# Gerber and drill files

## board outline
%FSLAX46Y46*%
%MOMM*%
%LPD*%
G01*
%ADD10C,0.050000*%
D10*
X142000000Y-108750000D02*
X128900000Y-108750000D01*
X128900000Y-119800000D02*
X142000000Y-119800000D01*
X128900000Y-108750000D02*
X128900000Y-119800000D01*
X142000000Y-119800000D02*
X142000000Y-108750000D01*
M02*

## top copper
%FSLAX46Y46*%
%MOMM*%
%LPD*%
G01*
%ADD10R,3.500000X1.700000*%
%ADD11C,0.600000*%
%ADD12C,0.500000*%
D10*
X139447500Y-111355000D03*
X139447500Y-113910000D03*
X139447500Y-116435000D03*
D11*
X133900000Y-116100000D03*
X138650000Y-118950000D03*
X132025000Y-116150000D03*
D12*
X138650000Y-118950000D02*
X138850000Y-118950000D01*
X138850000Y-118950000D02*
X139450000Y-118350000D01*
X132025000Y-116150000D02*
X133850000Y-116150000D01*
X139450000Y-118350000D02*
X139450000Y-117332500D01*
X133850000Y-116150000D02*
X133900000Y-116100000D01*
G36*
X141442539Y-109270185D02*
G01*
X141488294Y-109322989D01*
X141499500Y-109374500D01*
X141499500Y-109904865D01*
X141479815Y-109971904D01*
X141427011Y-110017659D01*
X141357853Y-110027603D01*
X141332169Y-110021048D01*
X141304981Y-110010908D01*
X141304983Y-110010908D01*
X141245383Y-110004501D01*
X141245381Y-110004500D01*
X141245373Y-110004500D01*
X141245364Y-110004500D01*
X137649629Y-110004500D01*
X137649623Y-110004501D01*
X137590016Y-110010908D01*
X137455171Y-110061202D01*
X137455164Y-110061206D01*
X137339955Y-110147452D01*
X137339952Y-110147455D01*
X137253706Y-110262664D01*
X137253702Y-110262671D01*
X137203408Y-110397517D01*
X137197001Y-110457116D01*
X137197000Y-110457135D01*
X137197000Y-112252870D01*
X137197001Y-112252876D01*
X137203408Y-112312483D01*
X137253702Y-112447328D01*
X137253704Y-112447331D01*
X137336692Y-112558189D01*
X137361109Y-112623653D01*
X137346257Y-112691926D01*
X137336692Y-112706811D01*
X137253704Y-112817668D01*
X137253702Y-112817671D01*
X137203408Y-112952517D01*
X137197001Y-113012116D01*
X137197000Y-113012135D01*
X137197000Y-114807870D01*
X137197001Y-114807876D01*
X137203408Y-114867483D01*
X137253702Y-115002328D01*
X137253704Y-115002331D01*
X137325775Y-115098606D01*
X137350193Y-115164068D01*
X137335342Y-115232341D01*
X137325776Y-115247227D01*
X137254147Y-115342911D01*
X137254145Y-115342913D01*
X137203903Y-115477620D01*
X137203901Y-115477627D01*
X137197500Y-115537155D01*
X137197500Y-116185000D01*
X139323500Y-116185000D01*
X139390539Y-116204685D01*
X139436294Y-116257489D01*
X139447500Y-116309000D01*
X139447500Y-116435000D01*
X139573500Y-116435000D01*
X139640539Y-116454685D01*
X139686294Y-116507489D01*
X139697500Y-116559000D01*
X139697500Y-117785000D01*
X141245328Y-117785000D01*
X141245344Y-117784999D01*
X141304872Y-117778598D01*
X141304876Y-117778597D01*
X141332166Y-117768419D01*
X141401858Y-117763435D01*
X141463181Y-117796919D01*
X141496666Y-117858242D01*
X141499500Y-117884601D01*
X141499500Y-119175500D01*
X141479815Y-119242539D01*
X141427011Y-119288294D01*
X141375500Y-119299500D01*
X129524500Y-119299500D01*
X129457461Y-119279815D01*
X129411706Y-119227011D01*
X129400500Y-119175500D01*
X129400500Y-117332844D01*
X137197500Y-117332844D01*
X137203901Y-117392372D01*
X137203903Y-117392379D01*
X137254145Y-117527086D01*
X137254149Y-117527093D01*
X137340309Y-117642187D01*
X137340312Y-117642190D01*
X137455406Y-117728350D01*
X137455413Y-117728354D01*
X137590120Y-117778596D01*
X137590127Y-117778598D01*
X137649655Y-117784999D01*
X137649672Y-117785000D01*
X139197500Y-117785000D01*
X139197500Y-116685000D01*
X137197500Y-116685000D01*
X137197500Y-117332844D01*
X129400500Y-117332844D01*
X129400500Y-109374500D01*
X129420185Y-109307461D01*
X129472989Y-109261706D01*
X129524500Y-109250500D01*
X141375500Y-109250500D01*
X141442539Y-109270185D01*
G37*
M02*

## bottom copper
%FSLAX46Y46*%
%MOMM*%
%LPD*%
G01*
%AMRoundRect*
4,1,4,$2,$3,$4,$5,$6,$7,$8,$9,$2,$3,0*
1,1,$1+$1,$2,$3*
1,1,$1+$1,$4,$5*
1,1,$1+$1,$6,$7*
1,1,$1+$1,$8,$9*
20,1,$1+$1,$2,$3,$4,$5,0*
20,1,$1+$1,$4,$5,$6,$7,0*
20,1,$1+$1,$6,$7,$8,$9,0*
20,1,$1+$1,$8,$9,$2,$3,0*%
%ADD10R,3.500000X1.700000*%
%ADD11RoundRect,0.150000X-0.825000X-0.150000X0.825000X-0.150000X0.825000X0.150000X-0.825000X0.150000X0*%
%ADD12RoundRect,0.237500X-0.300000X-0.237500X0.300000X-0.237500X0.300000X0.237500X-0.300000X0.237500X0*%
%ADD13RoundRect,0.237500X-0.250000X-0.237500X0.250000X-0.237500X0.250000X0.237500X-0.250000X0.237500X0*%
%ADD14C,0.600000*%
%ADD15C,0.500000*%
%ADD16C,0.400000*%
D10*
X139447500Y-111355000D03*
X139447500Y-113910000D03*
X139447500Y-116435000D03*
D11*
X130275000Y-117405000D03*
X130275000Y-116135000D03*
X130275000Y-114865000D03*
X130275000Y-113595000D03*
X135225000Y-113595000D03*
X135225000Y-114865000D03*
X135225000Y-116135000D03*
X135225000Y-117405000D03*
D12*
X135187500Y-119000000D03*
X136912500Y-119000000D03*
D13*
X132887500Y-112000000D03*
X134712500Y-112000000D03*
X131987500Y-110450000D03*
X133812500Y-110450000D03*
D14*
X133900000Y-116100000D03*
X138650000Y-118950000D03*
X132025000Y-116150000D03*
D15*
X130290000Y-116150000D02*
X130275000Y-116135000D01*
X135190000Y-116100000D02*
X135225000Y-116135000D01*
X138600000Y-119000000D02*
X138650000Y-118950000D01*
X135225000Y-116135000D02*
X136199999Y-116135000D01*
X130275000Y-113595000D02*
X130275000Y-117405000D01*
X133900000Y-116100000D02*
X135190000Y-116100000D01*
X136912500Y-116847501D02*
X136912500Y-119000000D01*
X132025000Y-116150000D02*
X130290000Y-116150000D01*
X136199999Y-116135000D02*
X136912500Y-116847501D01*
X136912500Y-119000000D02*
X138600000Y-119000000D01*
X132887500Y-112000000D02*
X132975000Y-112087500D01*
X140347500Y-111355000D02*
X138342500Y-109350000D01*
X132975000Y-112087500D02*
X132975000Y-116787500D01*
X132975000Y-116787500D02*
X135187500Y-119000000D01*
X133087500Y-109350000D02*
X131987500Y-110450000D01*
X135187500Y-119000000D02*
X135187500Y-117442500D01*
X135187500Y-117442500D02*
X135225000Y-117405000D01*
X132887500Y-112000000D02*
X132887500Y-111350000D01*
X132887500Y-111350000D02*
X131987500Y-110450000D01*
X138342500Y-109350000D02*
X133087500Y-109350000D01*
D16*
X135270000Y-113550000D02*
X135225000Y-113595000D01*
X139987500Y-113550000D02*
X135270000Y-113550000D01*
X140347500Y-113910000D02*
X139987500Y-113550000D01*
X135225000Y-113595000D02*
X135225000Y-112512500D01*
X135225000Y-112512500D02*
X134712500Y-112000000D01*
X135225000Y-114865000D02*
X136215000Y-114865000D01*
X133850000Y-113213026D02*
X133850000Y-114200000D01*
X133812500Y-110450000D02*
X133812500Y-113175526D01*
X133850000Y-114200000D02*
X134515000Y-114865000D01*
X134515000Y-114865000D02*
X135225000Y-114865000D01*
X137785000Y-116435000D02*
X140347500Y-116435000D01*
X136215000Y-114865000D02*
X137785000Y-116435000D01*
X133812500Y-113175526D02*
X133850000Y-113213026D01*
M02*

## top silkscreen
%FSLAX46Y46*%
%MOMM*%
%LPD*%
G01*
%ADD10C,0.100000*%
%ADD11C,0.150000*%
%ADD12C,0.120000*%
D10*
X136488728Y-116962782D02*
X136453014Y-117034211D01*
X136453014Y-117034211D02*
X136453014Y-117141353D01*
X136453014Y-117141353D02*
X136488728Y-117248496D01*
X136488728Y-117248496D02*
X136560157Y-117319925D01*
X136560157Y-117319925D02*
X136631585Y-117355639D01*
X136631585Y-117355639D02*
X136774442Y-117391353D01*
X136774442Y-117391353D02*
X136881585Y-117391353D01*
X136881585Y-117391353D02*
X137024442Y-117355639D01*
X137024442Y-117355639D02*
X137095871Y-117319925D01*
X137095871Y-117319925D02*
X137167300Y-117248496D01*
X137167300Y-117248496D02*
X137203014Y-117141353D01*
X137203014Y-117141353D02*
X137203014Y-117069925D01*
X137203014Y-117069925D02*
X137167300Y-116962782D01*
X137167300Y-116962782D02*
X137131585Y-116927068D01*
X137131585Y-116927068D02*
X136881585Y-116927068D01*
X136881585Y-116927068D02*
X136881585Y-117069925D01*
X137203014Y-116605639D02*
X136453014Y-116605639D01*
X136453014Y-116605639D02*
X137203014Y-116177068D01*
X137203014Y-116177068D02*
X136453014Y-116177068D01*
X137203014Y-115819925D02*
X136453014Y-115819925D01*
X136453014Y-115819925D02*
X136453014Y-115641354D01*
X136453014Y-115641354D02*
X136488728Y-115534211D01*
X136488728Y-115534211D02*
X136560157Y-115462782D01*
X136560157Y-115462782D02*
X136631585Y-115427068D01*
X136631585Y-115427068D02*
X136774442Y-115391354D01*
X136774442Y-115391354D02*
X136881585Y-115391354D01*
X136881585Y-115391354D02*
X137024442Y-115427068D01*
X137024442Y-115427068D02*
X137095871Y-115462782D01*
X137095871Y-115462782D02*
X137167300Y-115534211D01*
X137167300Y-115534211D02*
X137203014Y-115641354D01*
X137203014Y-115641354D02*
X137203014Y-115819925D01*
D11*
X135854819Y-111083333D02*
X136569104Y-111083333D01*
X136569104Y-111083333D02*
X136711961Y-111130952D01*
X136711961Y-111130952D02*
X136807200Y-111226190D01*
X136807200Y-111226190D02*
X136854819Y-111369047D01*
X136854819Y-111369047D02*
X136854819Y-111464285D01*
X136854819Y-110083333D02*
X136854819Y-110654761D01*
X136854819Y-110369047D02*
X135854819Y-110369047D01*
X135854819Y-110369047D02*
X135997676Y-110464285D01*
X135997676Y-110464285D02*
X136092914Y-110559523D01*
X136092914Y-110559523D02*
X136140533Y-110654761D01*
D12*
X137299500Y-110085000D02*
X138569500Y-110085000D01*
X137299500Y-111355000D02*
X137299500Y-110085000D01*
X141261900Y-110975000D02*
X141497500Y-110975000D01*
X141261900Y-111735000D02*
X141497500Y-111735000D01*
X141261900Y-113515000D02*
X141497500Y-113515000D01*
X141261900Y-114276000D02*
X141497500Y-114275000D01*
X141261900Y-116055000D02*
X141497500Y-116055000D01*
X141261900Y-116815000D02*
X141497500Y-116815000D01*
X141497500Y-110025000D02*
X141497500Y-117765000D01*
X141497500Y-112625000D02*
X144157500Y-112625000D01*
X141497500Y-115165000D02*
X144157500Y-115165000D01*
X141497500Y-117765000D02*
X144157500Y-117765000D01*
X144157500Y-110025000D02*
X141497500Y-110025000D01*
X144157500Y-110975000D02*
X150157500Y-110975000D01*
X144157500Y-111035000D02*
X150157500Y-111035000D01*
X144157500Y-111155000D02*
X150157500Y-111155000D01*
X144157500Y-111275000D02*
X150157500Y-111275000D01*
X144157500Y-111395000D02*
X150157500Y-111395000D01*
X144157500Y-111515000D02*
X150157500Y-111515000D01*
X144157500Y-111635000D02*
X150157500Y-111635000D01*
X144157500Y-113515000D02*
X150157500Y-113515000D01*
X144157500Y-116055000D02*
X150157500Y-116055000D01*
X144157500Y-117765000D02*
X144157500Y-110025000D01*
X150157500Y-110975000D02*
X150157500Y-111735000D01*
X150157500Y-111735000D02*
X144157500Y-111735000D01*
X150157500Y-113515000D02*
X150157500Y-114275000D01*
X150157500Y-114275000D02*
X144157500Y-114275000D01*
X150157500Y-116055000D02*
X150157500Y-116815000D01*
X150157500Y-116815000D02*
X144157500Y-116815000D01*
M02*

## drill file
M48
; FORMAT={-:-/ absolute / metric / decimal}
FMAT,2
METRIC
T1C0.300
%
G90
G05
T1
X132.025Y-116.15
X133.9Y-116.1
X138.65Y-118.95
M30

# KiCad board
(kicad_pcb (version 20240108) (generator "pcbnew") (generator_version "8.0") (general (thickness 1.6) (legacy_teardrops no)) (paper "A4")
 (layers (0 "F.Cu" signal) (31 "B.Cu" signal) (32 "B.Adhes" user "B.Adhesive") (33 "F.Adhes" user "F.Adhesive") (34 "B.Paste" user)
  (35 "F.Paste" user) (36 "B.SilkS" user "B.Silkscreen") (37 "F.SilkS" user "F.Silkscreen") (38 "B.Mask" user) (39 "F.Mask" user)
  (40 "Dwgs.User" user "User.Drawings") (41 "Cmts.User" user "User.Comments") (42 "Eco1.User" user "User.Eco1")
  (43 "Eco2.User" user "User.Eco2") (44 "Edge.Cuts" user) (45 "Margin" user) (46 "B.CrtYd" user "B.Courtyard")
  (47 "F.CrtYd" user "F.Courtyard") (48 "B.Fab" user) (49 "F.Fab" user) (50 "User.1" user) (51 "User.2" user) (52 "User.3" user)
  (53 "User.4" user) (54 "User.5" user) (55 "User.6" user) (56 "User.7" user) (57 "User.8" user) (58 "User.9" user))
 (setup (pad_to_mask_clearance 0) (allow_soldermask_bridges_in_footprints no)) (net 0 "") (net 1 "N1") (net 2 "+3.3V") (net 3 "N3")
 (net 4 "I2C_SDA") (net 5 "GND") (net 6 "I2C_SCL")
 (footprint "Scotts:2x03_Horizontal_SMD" (layer "F.Cu") (at 140.3475 108.815)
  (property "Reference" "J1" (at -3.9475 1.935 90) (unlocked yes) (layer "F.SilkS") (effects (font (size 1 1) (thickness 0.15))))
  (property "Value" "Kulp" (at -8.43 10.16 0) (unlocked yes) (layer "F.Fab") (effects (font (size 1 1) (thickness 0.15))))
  (fp_line (start -3.048 1.27) (end -1.778 1.27) (stroke (width 0.12) (type solid)) (layer "F.SilkS"))
  (fp_line (start -3.048 2.54) (end -3.048 1.27) (stroke (width 0.12) (type solid)) (layer "F.SilkS"))
  (fp_line (start 0.9144 2.16) (end 1.15 2.16) (stroke (width 0.12) (type solid)) (layer "F.SilkS"))
  (fp_line (start 0.9144 2.92) (end 1.15 2.92) (stroke (width 0.12) (type solid)) (layer "F.SilkS"))
  (fp_line (start 0.9144 4.7) (end 1.15 4.7) (stroke (width 0.12) (type solid)) (layer "F.SilkS"))
  (fp_line (start 0.9144 5.461) (end 1.15 5.46) (stroke (width 0.12) (type solid)) (layer "F.SilkS"))
  (fp_line (start 0.9144 7.24) (end 1.15 7.24) (stroke (width 0.12) (type solid)) (layer "F.SilkS"))
  (fp_line (start 0.9144 8) (end 1.15 8) (stroke (width 0.12) (type solid)) (layer "F.SilkS"))
  (fp_line (start 1.15 1.21) (end 1.15 8.95) (stroke (width 0.12) (type solid)) (layer "F.SilkS"))
  (fp_line (start 1.15 3.81) (end 3.81 3.81) (stroke (width 0.12) (type solid)) (layer "F.SilkS"))
  (fp_line (start 1.15 6.35) (end 3.81 6.35) (stroke (width 0.12) (type solid)) (layer "F.SilkS"))
  (fp_line (start 1.15 8.95) (end 3.81 8.95) (stroke (width 0.12) (type solid)) (layer "F.SilkS"))
  (fp_line (start 3.81 1.21) (end 1.15 1.21) (stroke (width 0.12) (type solid)) (layer "F.SilkS"))
  (fp_line (start 3.81 2.16) (end 9.81 2.16) (stroke (width 0.12) (type solid)) (layer "F.SilkS"))
  (fp_line (start 3.81 2.22) (end 9.81 2.22) (stroke (width 0.12) (type solid)) (layer "F.SilkS"))
  (fp_line (start 3.81 2.34) (end 9.81 2.34) (stroke (width 0.12) (type solid)) (layer "F.SilkS"))
  (fp_line (start 3.81 2.46) (end 9.81 2.46) (stroke (width 0.12) (type solid)) (layer "F.SilkS"))
  (fp_line (start 3.81 2.58) (end 9.81 2.58) (stroke (width 0.12) (type solid)) (layer "F.SilkS"))
  (fp_line (start 3.81 2.7) (end 9.81 2.7) (stroke (width 0.12) (type solid)) (layer "F.SilkS"))
  (fp_line (start 3.81 2.82) (end 9.81 2.82) (stroke (width 0.12) (type solid)) (layer "F.SilkS"))
  (fp_line (start 3.81 4.7) (end 9.81 4.7) (stroke (width 0.12) (type solid)) (layer "F.SilkS"))
  (fp_line (start 3.81 7.24) (end 9.81 7.24) (stroke (width 0.12) (type solid)) (layer "F.SilkS"))
  (fp_line (start 3.81 8.95) (end 3.81 1.21) (stroke (width 0.12) (type solid)) (layer "F.SilkS"))
  (fp_line (start 9.81 2.16) (end 9.81 2.92) (stroke (width 0.12) (type solid)) (layer "F.SilkS"))
  (fp_line (start 9.81 2.92) (end 3.81 2.92) (stroke (width 0.12) (type solid)) (layer "F.SilkS"))
  (fp_line (start 9.81 4.7) (end 9.81 5.46) (stroke (width 0.12) (type solid)) (layer "F.SilkS"))
  (fp_line (start 9.81 5.46) (end 3.81 5.46) (stroke (width 0.12) (type solid)) (layer "F.SilkS"))
  (fp_line (start 9.81 7.24) (end 9.81 8) (stroke (width 0.12) (type solid)) (layer "F.SilkS"))
  (fp_line (start 9.81 8) (end 3.81 8) (stroke (width 0.12) (type solid)) (layer "F.SilkS"))
  (pad "1" smd rect (at 0 2.54) (size 3.5 1.7) (drill (offset -0.9 0)) (layers "F.Cu" "F.Mask") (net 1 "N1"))
  (pad "2" smd rect (at 0 2.54) (size 3.5 1.7) (drill (offset -0.9 0)) (layers "B.Cu" "B.Mask") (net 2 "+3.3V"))
  (pad "3" smd rect (at 0 5.095) (size 3.5 1.7) (drill (offset -0.9 0)) (layers "F.Cu" "F.Mask") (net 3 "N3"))
  (pad "4" smd rect (at 0 5.095) (size 3.5 1.7) (drill (offset -0.9 0)) (layers "B.Cu" "B.Mask") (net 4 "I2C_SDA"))
  (pad "5" smd rect (at 0 7.62) (size 3.5 1.7) (drill (offset -0.9 0)) (layers "F.Cu" "F.Mask") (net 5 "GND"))
  (pad "6" smd rect (at 0 7.62) (size 3.5 1.7) (drill (offset -0.9 0)) (layers "B.Cu" "B.Mask") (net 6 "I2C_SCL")))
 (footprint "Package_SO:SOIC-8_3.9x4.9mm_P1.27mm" (layer "B.Cu") (at 132.75 115.5)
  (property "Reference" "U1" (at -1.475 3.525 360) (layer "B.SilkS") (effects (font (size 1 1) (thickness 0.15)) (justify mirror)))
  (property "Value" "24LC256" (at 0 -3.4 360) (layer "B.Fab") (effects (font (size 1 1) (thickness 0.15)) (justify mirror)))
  (pad "1" smd roundrect (at -2.475 1.905) (size 1.95 0.6) (layers "B.Cu" "B.Paste" "B.Mask") (roundrect_rratio 0.25) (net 5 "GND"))
  (pad "2" smd roundrect (at -2.475 0.635) (size 1.95 0.6) (layers "B.Cu" "B.Paste" "B.Mask") (roundrect_rratio 0.25) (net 5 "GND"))
  (pad "3" smd roundrect (at -2.475 -0.635) (size 1.95 0.6) (layers "B.Cu" "B.Paste" "B.Mask") (roundrect_rratio 0.25) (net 5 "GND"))
  (pad "4" smd roundrect (at -2.475 -1.905) (size 1.95 0.6) (layers "B.Cu" "B.Paste" "B.Mask") (roundrect_rratio 0.25) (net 5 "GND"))
  (pad "5" smd roundrect (at 2.475 -1.905) (size 1.95 0.6) (layers "B.Cu" "B.Paste" "B.Mask") (roundrect_rratio 0.25) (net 4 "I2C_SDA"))
  (pad "6" smd roundrect (at 2.475 -0.635) (size 1.95 0.6) (layers "B.Cu" "B.Paste" "B.Mask") (roundrect_rratio 0.25) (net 6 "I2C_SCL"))
  (pad "7" smd roundrect (at 2.475 0.635) (size 1.95 0.6) (layers "B.Cu" "B.Paste" "B.Mask") (roundrect_rratio 0.25) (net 5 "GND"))
  (pad "8" smd roundrect (at 2.475 1.905) (size 1.95 0.6) (layers "B.Cu" "B.Paste" "B.Mask") (roundrect_rratio 0.25) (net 2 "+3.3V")))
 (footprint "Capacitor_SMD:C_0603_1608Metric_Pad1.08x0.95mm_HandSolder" (layer "B.Cu") (at 136.05 119)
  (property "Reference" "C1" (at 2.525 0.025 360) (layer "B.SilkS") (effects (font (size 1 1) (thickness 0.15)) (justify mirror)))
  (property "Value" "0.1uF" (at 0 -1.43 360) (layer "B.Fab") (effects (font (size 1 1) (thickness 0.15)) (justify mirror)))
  (pad "1" smd roundrect (at -0.8625 0) (size 1.075 0.95) (layers "B.Cu" "B.Paste" "B.Mask") (roundrect_rratio 0.25) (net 2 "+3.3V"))
  (pad "2" smd roundrect (at 0.8625 0) (size 1.075 0.95) (layers "B.Cu" "B.Paste" "B.Mask") (roundrect_rratio 0.25) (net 5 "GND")))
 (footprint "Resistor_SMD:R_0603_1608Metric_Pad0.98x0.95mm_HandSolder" (layer "B.Cu") (at 133.8 112)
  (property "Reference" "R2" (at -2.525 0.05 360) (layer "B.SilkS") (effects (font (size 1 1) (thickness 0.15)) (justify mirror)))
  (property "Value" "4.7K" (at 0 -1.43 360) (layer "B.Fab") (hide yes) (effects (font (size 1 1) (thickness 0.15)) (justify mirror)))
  (pad "1" smd roundrect (at -0.9125 0) (size 0.975 0.95) (layers "B.Cu" "B.Paste" "B.Mask") (roundrect_rratio 0.25) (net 2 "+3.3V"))
  (pad "2" smd roundrect (at 0.9125 0) (size 0.975 0.95) (layers "B.Cu" "B.Paste" "B.Mask") (roundrect_rratio 0.25) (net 4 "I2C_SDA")))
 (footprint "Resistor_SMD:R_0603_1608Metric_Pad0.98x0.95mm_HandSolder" (layer "B.Cu") (at 132.9 110.45)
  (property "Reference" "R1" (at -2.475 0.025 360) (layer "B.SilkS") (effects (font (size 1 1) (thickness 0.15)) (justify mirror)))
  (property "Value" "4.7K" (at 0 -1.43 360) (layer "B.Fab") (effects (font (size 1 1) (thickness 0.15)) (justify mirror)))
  (pad "1" smd roundrect (at -0.9125 0) (size 0.975 0.95) (layers "B.Cu" "B.Paste" "B.Mask") (roundrect_rratio 0.25) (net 2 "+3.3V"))
  (pad "2" smd roundrect (at 0.9125 0) (size 0.975 0.95) (layers "B.Cu" "B.Paste" "B.Mask") (roundrect_rratio 0.25) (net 6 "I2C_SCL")))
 (gr_line (start 142 108.75) (end 128.9 108.75) (stroke (width 0.05) (type default)) (layer "Edge.Cuts"))
 (gr_line (start 128.9 119.8) (end 142 119.8) (stroke (width 0.05) (type default)) (layer "Edge.Cuts"))
 (gr_line (start 128.9 108.75) (end 128.9 119.8) (stroke (width 0.05) (type default)) (layer "Edge.Cuts"))
 (gr_line (start 142 119.8) (end 142 108.75) (stroke (width 0.05) (type default)) (layer "Edge.Cuts"))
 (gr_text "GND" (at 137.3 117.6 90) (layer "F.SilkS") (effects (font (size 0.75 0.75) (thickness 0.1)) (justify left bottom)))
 (segment (start 138.65 118.95) (end 138.85 118.95) (width 0.5) (layer "F.Cu") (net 5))
 (segment (start 138.85 118.95) (end 139.45 118.35) (width 0.5) (layer "F.Cu") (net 5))
 (segment (start 132.025 116.15) (end 133.85 116.15) (width 0.5) (layer "F.Cu") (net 5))
 (segment (start 139.45 118.35) (end 139.45 117.3325) (width 0.5) (layer "F.Cu") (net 5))
 (segment (start 133.85 116.15) (end 133.9 116.1) (width 0.5) (layer "F.Cu") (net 5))
 (via (at 133.9 116.1) (size 0.6) (drill 0.3) (layers "F.Cu" "B.Cu") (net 5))
 (via (at 138.65 118.95) (size 0.6) (drill 0.3) (layers "F.Cu" "B.Cu") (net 5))
 (via (at 132.025 116.15) (size 0.6) (drill 0.3) (layers "F.Cu" "B.Cu") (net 5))
 (segment (start 130.29 116.15) (end 130.275 116.135) (width 0.5) (layer "B.Cu") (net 5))
 (segment (start 135.19 116.1) (end 135.225 116.135) (width 0.5) (layer "B.Cu") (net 5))
 (segment (start 138.6 119) (end 138.65 118.95) (width 0.5) (layer "B.Cu") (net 5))
 (segment (start 135.225 116.135) (end 136.199999 116.135) (width 0.5) (layer "B.Cu") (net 5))
 (segment (start 130.275 113.595) (end 130.275 117.405) (width 0.5) (layer "B.Cu") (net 5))
 (segment (start 133.9 116.1) (end 135.19 116.1) (width 0.5) (layer "B.Cu") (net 5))
 (segment (start 136.9125 116.847501) (end 136.9125 119) (width 0.5) (layer "B.Cu") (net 5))
 (segment (start 132.025 116.15) (end 130.29 116.15) (width 0.5) (layer "B.Cu") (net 5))
 (segment (start 136.199999 116.135) (end 136.9125 116.847501) (width 0.5) (layer "B.Cu") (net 5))
 (segment (start 136.9125 119) (end 138.6 119) (width 0.5) (layer "B.Cu") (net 5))
 (segment (start 132.8875 112) (end 132.975 112.0875) (width 0.5) (layer "B.Cu") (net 2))
 (segment (start 140.3475 111.355) (end 138.3425 109.35) (width 0.5) (layer "B.Cu") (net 2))
 (segment (start 132.975 112.0875) (end 132.975 116.7875) (width 0.5) (layer "B.Cu") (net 2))
 (segment (start 132.975 116.7875) (end 135.1875 119) (width 0.5) (layer "B.Cu") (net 2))
 (segment (start 133.0875 109.35) (end 131.9875 110.45) (width 0.5) (layer "B.Cu") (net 2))
 (segment (start 135.1875 119) (end 135.1875 117.4425) (width 0.5) (layer "B.Cu") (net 2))
 (segment (start 135.1875 117.4425) (end 135.225 117.405) (width 0.5) (layer "B.Cu") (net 2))
 (segment (start 132.8875 112) (end 132.8875 111.35) (width 0.5) (layer "B.Cu") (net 2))
 (segment (start 132.8875 111.35) (end 131.9875 110.45) (width 0.5) (layer "B.Cu") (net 2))
 (segment (start 138.3425 109.35) (end 133.0875 109.35) (width 0.5) (layer "B.Cu") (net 2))
 (segment (start 135.27 113.55) (end 135.225 113.595) (width 0.4) (layer "B.Cu") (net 4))
 (segment (start 139.9875 113.55) (end 135.27 113.55) (width 0.4) (layer "B.Cu") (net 4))
 (segment (start 140.3475 113.91) (end 139.9875 113.55) (width 0.4) (layer "B.Cu") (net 4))
 (segment (start 135.225 113.595) (end 135.225 112.5125) (width 0.4) (layer "B.Cu") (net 4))
 (segment (start 135.225 112.5125) (end 134.7125 112) (width 0.4) (layer "B.Cu") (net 4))
 (segment (start 135.225 114.865) (end 136.215 114.865) (width 0.4) (layer "B.Cu") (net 6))
 (segment (start 133.85 113.213026) (end 133.85 114.2) (width 0.4) (layer "B.Cu") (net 6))
 (segment (start 133.8125 110.45) (end 133.8125 113.175526) (width 0.4) (layer "B.Cu") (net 6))
 (segment (start 133.85 114.2) (end 134.515 114.865) (width 0.4) (layer "B.Cu") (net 6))
 (segment (start 134.515 114.865) (end 135.225 114.865) (width 0.4) (layer "B.Cu") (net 6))
 (segment (start 137.785 116.435) (end 140.3475 116.435) (width 0.4) (layer "B.Cu") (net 6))
 (segment (start 136.215 114.865) (end 137.785 116.435) (width 0.4) (layer "B.Cu") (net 6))
 (segment (start 133.8125 113.175526) (end 133.85 113.213026) (width 0.4) (layer "B.Cu") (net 6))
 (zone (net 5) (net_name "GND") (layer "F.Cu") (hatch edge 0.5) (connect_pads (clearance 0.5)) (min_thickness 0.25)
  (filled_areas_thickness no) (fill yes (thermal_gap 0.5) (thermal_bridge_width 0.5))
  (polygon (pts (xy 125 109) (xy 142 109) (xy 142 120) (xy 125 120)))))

